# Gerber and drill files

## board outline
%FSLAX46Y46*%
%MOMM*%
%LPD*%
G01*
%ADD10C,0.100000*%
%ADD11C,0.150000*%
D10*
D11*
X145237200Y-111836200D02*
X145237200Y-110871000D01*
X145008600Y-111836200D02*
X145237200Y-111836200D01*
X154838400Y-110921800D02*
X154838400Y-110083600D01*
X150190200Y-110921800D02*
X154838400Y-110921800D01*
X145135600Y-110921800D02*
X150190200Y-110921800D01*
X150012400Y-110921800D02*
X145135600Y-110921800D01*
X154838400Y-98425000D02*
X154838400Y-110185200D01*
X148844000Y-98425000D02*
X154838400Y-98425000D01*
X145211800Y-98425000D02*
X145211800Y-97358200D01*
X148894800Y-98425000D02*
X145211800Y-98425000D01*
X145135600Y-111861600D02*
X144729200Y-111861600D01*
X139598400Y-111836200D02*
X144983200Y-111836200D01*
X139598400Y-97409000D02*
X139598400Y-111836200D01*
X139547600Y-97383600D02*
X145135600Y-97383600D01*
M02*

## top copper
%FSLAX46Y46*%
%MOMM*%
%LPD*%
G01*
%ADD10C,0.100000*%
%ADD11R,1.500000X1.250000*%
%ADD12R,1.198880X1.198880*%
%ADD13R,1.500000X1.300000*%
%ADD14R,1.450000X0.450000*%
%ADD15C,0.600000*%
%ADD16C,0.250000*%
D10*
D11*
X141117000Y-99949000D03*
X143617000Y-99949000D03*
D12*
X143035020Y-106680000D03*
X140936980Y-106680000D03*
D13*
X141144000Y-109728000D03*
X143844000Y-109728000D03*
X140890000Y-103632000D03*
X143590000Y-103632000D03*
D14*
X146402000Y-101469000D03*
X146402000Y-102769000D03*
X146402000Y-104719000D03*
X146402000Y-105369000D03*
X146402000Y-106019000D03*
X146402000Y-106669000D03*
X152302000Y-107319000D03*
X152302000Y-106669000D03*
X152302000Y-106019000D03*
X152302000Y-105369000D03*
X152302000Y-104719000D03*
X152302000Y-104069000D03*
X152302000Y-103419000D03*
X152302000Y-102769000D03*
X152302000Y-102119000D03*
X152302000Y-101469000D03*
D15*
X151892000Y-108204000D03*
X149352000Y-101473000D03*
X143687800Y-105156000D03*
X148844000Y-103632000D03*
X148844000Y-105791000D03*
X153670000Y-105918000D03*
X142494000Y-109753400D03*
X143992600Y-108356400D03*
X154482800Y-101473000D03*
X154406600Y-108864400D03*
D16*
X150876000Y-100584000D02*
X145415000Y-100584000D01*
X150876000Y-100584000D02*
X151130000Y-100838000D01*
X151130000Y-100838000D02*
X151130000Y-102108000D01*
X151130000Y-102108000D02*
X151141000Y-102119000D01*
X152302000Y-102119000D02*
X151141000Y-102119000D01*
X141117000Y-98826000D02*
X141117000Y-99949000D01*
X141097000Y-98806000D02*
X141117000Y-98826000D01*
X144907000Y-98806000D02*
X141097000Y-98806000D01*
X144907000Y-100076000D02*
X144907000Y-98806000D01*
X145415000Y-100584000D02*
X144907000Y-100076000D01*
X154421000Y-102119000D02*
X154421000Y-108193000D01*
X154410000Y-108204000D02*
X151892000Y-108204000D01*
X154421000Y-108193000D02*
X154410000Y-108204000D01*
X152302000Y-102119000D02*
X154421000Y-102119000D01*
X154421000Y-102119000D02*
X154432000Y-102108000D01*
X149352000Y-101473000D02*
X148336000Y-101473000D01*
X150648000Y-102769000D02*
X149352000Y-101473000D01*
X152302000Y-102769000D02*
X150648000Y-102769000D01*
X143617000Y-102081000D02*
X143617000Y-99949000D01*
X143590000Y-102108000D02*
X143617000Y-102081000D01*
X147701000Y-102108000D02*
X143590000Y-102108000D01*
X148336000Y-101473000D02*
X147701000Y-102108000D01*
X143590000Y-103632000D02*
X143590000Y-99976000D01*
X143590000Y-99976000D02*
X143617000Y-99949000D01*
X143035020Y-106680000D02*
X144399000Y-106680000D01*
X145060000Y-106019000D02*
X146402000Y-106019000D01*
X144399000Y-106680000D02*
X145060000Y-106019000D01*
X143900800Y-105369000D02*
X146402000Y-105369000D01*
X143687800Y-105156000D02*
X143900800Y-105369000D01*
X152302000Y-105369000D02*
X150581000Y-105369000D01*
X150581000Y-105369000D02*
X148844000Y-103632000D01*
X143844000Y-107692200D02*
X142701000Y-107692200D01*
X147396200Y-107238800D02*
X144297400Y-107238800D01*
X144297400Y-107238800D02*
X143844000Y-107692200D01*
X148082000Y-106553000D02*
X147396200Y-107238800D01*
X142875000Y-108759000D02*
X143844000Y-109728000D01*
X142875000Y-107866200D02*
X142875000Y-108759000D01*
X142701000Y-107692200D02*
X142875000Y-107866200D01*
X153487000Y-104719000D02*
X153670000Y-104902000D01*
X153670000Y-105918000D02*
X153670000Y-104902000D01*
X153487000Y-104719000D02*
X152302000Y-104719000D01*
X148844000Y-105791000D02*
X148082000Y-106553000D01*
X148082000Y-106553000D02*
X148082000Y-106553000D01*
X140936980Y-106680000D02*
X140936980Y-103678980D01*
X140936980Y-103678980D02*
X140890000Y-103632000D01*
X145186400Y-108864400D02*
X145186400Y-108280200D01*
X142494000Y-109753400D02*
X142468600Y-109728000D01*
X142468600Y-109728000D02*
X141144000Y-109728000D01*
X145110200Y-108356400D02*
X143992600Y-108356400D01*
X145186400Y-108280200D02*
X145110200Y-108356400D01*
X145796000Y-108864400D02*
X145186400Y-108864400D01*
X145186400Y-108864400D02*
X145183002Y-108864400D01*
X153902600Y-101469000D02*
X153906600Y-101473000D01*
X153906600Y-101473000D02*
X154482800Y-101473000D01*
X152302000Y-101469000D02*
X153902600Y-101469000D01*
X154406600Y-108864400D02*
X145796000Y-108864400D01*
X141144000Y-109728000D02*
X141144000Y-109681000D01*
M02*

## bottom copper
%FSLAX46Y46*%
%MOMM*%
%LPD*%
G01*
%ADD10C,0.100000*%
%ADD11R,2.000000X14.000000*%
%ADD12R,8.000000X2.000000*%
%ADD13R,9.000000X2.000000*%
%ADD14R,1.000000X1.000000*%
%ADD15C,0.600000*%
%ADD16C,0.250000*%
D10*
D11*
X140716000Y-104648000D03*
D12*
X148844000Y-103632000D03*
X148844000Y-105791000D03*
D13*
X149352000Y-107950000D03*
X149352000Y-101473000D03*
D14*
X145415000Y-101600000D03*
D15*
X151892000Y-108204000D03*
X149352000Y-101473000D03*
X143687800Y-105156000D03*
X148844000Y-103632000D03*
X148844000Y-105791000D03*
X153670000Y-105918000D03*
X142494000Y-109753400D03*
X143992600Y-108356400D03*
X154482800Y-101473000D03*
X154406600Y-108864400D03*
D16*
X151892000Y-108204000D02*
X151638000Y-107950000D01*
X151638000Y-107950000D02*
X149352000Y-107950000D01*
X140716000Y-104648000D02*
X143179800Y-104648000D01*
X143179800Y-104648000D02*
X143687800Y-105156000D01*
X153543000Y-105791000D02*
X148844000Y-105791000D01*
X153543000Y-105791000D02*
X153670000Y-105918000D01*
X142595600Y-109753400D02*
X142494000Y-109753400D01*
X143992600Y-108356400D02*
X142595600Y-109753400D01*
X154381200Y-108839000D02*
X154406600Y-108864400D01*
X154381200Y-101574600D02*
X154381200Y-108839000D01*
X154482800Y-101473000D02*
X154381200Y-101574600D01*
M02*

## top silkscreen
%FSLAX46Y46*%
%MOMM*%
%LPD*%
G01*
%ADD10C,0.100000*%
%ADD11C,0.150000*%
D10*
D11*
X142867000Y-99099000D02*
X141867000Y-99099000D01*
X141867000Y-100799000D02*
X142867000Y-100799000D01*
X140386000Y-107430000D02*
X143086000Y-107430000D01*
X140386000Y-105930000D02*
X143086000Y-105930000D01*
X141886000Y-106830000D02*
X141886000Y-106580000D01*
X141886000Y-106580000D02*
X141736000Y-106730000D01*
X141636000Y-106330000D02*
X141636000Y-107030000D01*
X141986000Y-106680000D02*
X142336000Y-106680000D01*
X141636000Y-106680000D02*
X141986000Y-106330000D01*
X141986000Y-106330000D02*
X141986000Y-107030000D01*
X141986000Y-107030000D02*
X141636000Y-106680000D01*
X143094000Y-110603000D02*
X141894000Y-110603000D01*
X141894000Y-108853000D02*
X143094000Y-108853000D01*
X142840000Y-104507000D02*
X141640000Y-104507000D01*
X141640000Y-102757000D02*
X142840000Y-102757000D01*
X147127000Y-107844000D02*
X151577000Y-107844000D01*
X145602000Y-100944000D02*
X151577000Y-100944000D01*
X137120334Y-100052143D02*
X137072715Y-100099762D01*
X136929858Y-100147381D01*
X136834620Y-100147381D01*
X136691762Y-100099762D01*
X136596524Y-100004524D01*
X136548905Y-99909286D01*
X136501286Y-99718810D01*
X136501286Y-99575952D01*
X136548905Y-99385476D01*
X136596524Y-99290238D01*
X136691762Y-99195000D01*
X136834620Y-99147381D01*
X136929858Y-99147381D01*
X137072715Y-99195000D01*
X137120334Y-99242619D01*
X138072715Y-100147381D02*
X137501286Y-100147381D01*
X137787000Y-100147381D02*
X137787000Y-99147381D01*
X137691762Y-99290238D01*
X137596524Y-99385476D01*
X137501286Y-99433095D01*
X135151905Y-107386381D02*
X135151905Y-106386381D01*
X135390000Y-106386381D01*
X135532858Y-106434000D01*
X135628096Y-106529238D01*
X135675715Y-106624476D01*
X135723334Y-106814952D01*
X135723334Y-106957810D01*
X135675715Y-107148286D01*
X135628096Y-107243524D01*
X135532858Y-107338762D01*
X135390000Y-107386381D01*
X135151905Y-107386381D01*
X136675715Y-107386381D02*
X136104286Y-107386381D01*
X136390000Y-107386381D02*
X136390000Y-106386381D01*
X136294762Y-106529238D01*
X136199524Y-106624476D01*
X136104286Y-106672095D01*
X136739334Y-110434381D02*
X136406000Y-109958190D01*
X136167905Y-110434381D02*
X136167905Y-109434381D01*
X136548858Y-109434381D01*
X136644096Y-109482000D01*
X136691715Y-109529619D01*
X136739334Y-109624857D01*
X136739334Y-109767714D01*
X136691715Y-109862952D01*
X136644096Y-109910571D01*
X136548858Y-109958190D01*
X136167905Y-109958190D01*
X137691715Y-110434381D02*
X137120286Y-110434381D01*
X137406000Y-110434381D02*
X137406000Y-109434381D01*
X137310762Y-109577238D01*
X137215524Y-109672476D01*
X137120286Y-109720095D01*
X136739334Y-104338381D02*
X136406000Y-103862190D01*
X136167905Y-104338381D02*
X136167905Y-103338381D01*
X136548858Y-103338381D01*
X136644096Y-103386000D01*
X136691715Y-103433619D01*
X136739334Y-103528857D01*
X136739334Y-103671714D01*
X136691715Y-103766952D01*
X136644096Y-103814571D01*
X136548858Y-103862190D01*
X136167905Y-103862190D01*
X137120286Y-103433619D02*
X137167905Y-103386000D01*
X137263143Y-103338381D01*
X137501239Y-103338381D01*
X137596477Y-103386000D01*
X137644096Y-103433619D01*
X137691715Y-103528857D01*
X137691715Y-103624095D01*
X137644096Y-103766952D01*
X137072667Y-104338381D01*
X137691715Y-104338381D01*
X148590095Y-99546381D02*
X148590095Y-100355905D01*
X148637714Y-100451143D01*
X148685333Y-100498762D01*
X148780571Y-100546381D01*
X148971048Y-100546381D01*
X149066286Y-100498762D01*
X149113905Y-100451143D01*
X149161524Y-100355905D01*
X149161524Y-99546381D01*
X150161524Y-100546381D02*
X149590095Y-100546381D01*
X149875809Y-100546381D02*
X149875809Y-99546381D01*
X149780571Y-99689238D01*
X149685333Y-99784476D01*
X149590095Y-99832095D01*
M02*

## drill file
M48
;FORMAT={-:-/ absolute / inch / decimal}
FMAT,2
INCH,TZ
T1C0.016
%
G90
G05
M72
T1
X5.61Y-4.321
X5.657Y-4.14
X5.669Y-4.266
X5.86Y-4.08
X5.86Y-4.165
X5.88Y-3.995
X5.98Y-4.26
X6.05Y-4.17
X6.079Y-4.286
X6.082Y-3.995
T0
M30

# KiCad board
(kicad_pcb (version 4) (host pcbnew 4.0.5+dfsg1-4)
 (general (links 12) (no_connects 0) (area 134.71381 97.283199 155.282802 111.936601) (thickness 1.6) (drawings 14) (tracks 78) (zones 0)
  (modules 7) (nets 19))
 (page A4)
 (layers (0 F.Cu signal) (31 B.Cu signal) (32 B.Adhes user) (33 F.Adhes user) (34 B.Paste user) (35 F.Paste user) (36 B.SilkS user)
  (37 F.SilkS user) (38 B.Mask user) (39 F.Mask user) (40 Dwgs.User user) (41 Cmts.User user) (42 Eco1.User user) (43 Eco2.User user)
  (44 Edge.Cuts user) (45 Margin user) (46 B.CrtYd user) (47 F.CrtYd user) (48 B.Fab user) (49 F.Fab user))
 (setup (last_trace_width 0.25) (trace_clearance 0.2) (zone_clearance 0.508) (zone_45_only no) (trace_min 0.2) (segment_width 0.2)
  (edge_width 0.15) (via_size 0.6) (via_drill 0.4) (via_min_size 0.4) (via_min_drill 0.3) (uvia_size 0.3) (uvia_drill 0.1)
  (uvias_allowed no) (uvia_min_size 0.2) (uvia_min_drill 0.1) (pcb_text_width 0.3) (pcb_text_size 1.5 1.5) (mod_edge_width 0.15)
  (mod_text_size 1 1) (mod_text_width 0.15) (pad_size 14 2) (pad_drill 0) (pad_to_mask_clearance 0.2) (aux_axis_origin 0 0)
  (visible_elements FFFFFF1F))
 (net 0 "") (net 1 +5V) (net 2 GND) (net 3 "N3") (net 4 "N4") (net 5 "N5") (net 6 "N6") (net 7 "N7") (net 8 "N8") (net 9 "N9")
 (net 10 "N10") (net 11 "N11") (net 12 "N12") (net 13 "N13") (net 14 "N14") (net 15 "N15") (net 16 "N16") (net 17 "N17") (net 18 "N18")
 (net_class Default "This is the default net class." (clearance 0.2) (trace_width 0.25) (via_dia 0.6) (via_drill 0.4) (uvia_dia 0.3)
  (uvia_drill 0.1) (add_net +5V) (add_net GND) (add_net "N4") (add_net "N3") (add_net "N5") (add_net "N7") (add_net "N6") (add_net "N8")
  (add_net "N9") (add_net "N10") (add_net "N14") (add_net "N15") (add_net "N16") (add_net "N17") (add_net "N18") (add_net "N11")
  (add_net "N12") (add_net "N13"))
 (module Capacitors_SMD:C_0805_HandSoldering (layer F.Cu) (at 142.367 99.949)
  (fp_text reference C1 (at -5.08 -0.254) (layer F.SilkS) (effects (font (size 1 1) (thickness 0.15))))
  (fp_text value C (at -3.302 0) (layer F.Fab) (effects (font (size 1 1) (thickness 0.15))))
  (fp_line (start 0.5 -0.85) (end -0.5 -0.85) (layer F.SilkS) (width 0.15))
  (fp_line (start -0.5 0.85) (end 0.5 0.85) (layer F.SilkS) (width 0.15))
  (pad 1 smd rect (at -1.25 0) (size 1.5 1.25) (layers F.Cu F.Paste F.Mask) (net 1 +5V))
  (pad 2 smd rect (at 1.25 0) (size 1.5 1.25) (layers F.Cu F.Paste F.Mask) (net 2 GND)))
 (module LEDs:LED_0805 (layer F.Cu) (at 141.986 106.68)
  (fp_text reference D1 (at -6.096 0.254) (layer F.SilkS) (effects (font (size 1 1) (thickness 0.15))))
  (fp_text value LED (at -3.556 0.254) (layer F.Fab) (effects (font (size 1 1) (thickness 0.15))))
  (fp_line (start -1.6 0.75) (end 1.1 0.75) (layer F.SilkS) (width 0.15))
  (fp_line (start -1.6 -0.75) (end 1.1 -0.75) (layer F.SilkS) (width 0.15))
  (fp_line (start -0.1 0.15) (end -0.1 -0.1) (layer F.SilkS) (width 0.15))
  (fp_line (start -0.1 -0.1) (end -0.25 0.05) (layer F.SilkS) (width 0.15))
  (fp_line (start -0.35 -0.35) (end -0.35 0.35) (layer F.SilkS) (width 0.15))
  (fp_line (start 0 0) (end 0.35 0) (layer F.SilkS) (width 0.15))
  (fp_line (start -0.35 0) (end 0 -0.35) (layer F.SilkS) (width 0.15))
  (fp_line (start 0 -0.35) (end 0 0.35) (layer F.SilkS) (width 0.15))
  (fp_line (start 0 0.35) (end -0.35 0) (layer F.SilkS) (width 0.15))
  (pad 2 smd rect (at 1.04902 0 180) (size 1.19888 1.19888) (layers F.Cu F.Paste F.Mask) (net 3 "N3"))
  (pad 1 smd rect (at -1.04902 0 180) (size 1.19888 1.19888) (layers F.Cu F.Paste F.Mask) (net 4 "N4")))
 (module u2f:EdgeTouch (layer B.Cu) (at 140.716 104.648 270)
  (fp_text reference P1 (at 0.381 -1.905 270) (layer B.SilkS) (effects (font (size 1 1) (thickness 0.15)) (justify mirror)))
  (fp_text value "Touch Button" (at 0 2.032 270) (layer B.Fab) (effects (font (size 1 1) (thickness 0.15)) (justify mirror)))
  (pad 1 connect rect (at 0 0 270) (size 14 2) (layers B.Cu B.Mask) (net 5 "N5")))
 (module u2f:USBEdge (layer B.Cu) (at 148.844 104.648)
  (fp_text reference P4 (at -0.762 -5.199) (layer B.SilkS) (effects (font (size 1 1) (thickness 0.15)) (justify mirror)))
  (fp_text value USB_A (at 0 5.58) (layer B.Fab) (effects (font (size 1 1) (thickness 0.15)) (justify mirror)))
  (pad 3 connect rect (at 0 -1.016) (size 8 2) (layers B.Cu B.Mask) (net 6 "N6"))
  (pad 2 connect rect (at 0 1.143) (size 8 2) (layers B.Cu B.Mask) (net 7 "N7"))
  (pad 1 connect rect (at 0.508 3.302) (size 9 2) (layers B.Cu B.Mask) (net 1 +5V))
  (pad 4 connect rect (at 0.508 -3.175) (size 9 2) (layers B.Cu B.Mask) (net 2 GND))
  (pad 5 connect rect (at -3.429 -3.048) (size 1 1) (layers B.Cu B.Mask) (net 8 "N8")))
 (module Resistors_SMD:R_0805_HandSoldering (layer F.Cu) (at 142.494 109.728)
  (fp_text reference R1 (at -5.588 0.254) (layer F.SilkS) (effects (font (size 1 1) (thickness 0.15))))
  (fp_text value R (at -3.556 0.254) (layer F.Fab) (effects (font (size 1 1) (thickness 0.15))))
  (fp_line (start 0.6 0.875) (end -0.6 0.875) (layer F.SilkS) (width 0.15))
  (fp_line (start -0.6 -0.875) (end 0.6 -0.875) (layer F.SilkS) (width 0.15))
  (pad 1 smd rect (at -1.35 0) (size 1.5 1.3) (layers F.Cu F.Paste F.Mask) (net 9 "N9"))
  (pad 2 smd rect (at 1.35 0) (size 1.5 1.3) (layers F.Cu F.Paste F.Mask) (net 7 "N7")))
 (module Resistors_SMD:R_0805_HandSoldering (layer F.Cu) (at 142.24 103.632)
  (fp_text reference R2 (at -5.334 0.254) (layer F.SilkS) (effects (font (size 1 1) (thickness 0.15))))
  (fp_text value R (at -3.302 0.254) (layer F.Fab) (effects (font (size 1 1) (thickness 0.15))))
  (fp_line (start 0.6 0.875) (end -0.6 0.875) (layer F.SilkS) (width 0.15))
  (fp_line (start -0.6 -0.875) (end 0.6 -0.875) (layer F.SilkS) (width 0.15))
  (pad 1 smd rect (at -1.35 0) (size 1.5 1.3) (layers F.Cu F.Paste F.Mask) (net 4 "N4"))
  (pad 2 smd rect (at 1.35 0) (size 1.5 1.3) (layers F.Cu F.Paste F.Mask) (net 2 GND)))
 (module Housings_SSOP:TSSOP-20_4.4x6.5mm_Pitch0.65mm (layer F.Cu) (at 149.352 104.394)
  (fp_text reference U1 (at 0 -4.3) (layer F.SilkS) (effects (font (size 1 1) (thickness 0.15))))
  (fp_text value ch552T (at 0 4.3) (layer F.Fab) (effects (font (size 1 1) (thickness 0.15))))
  (fp_line (start -2.225 3.45) (end 2.225 3.45) (layer F.SilkS) (width 0.15))
  (fp_line (start -3.75 -3.45) (end 2.225 -3.45) (layer F.SilkS) (width 0.15))
  (pad 1 smd rect (at -2.95 -2.925) (size 1.45 0.45) (layers F.Cu F.Paste F.Mask) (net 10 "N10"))
  (pad 3 smd rect (at -2.95 -1.625) (size 1.45 0.45) (layers F.Cu F.Paste F.Mask) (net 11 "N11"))
  (pad 6 smd rect (at -2.95 0.325) (size 1.45 0.45) (layers F.Cu F.Paste F.Mask) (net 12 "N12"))
  (pad 7 smd rect (at -2.95 0.975) (size 1.45 0.45) (layers F.Cu F.Paste F.Mask) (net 5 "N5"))
  (pad 8 smd rect (at -2.95 1.625) (size 1.45 0.45) (layers F.Cu F.Paste F.Mask) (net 3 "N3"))
  (pad 9 smd rect (at -2.95 2.275) (size 1.45 0.45) (layers F.Cu F.Paste F.Mask) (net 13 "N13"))
  (pad 11 smd rect (at 2.95 2.925) (size 1.45 0.45) (layers F.Cu F.Paste F.Mask) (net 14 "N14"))
  (pad 12 smd rect (at 2.95 2.275) (size 1.45 0.45) (layers F.Cu F.Paste F.Mask) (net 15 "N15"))
  (pad 13 smd rect (at 2.95 1.625) (size 1.45 0.45) (layers F.Cu F.Paste F.Mask) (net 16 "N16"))
  (pad 14 smd rect (at 2.95 0.975) (size 1.45 0.45) (layers F.Cu F.Paste F.Mask) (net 6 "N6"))
  (pad 15 smd rect (at 2.95 0.325) (size 1.45 0.45) (layers F.Cu F.Paste F.Mask) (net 7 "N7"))
  (pad 16 smd rect (at 2.95 -0.325) (size 1.45 0.45) (layers F.Cu F.Paste F.Mask) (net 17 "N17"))
  (pad 17 smd rect (at 2.95 -0.975) (size 1.45 0.45) (layers F.Cu F.Paste F.Mask) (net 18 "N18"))
  (pad 18 smd rect (at 2.95 -1.625) (size 1.45 0.45) (layers F.Cu F.Paste F.Mask) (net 2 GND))
  (pad 19 smd rect (at 2.95 -2.275) (size 1.45 0.45) (layers F.Cu F.Paste F.Mask) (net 1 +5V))
  (pad 20 smd rect (at 2.95 -2.925) (size 1.45 0.45) (layers F.Cu F.Paste F.Mask) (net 9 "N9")))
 (gr_line (start 145.2372 111.8362) (end 145.2372 110.871) (angle 90) (layer Edge.Cuts) (width 0.15))
 (gr_line (start 145.0086 111.8362) (end 145.2372 111.8362) (angle 90) (layer Edge.Cuts) (width 0.15))
 (gr_line (start 154.8384 110.9218) (end 154.8384 110.0836) (angle 90) (layer Edge.Cuts) (width 0.15))
 (gr_line (start 150.1902 110.9218) (end 154.8384 110.9218) (angle 90) (layer Edge.Cuts) (width 0.15))
 (gr_line (start 145.1356 110.9218) (end 150.1902 110.9218) (angle 90) (layer Edge.Cuts) (width 0.15))
 (gr_line (start 150.0124 110.9218) (end 145.1356 110.9218) (angle 90) (layer Edge.Cuts) (width 0.15))
 (gr_line (start 154.8384 98.425) (end 154.8384 110.1852) (angle 90) (layer Edge.Cuts) (width 0.15))
 (gr_line (start 148.844 98.425) (end 154.8384 98.425) (angle 90) (layer Edge.Cuts) (width 0.15))
 (gr_line (start 145.2118 98.425) (end 145.2118 97.3582) (angle 90) (layer Edge.Cuts) (width 0.15))
 (gr_line (start 148.8948 98.425) (end 145.2118 98.425) (angle 90) (layer Edge.Cuts) (width 0.15))
 (gr_line (start 145.1356 111.8616) (end 144.7292 111.8616) (angle 90) (layer Edge.Cuts) (width 0.15))
 (gr_line (start 139.5984 111.8362) (end 144.9832 111.8362) (angle 90) (layer Edge.Cuts) (width 0.15))
 (gr_line (start 139.5984 97.409) (end 139.5984 111.8362) (angle 90) (layer Edge.Cuts) (width 0.15))
 (gr_line (start 139.5476 97.3836) (end 145.1356 97.3836) (angle 90) (layer Edge.Cuts) (width 0.15))
 (segment (start 150.876 100.584) (end 145.415 100.584) (width 0.25) (layer F.Cu) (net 1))
 (segment (start 150.876 100.584) (end 151.13 100.838) (width 0.25) (layer F.Cu) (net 1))
 (segment (start 151.13 100.838) (end 151.13 102.108) (width 0.25) (layer F.Cu) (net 1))
 (segment (start 151.13 102.108) (end 151.141 102.119) (width 0.25) (layer F.Cu) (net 1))
 (segment (start 152.302 102.119) (end 151.141 102.119) (width 0.25) (layer F.Cu) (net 1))
 (segment (start 141.117 98.826) (end 141.117 99.949) (width 0.25) (layer F.Cu) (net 1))
 (segment (start 141.097 98.806) (end 141.117 98.826) (width 0.25) (layer F.Cu) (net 1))
 (segment (start 144.907 98.806) (end 141.097 98.806) (width 0.25) (layer F.Cu) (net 1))
 (segment (start 144.907 100.076) (end 144.907 98.806) (width 0.25) (layer F.Cu) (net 1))
 (segment (start 145.415 100.584) (end 144.907 100.076) (width 0.25) (layer F.Cu) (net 1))
 (segment (start 154.421 102.119) (end 154.421 108.193) (width 0.25) (layer F.Cu) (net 1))
 (segment (start 151.892 108.204) (end 151.638 107.95) (width 0.25) (layer B.Cu) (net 1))
 (via (at 151.892 108.204) (size 0.6) (drill 0.4) (layers F.Cu B.Cu) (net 1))
 (segment (start 154.41 108.204) (end 151.892 108.204) (width 0.25) (layer F.Cu) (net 1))
 (segment (start 154.421 108.193) (end 154.41 108.204) (width 0.25) (layer F.Cu) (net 1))
 (segment (start 151.638 107.95) (end 149.352 107.95) (width 0.25) (layer B.Cu) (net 1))
 (segment (start 152.302 102.119) (end 154.421 102.119) (width 0.25) (layer F.Cu) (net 1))
 (segment (start 154.421 102.119) (end 154.432 102.108) (width 0.25) (layer F.Cu) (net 1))
 (segment (start 149.352 101.473) (end 148.336 101.473) (width 0.25) (layer F.Cu) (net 2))
 (segment (start 150.648 102.769) (end 149.352 101.473) (width 0.25) (layer F.Cu) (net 2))
 (segment (start 152.302 102.769) (end 150.648 102.769) (width 0.25) (layer F.Cu) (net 2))
 (via (at 149.352 101.473) (size 0.6) (drill 0.4) (layers F.Cu B.Cu) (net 2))
 (segment (start 143.617 102.081) (end 143.617 99.949) (width 0.25) (layer F.Cu) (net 2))
 (segment (start 143.59 102.108) (end 143.617 102.081) (width 0.25) (layer F.Cu) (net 2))
 (segment (start 147.701 102.108) (end 143.59 102.108) (width 0.25) (layer F.Cu) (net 2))
 (segment (start 148.336 101.473) (end 147.701 102.108) (width 0.25) (layer F.Cu) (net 2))
 (segment (start 143.59 103.632) (end 143.59 99.976) (width 0.25) (layer F.Cu) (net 2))
 (segment (start 143.59 99.976) (end 143.617 99.949) (width 0.25) (layer F.Cu) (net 2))
 (segment (start 143.03502 106.68) (end 144.399 106.68) (width 0.25) (layer F.Cu) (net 3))
 (segment (start 145.06 106.019) (end 146.402 106.019) (width 0.25) (layer F.Cu) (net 3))
 (segment (start 144.399 106.68) (end 145.06 106.019) (width 0.25) (layer F.Cu) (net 3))
 (segment (start 140.716 104.648) (end 143.1798 104.648) (width 0.25) (layer B.Cu) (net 5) (status 400000))
 (segment (start 143.9008 105.369) (end 146.402 105.369) (width 0.25) (layer F.Cu) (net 5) (status 800000))
 (segment (start 143.6878 105.156) (end 143.9008 105.369) (width 0.25) (layer F.Cu) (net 5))
 (via (at 143.6878 105.156) (size 0.6) (drill 0.4) (layers F.Cu B.Cu) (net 5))
 (segment (start 143.1798 104.648) (end 143.6878 105.156) (width 0.25) (layer B.Cu) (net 5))
 (via (at 148.844 103.632) (size 0.6) (drill 0.4) (layers F.Cu B.Cu) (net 6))
 (segment (start 152.302 105.369) (end 150.581 105.369) (width 0.25) (layer F.Cu) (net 6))
 (segment (start 150.581 105.369) (end 148.844 103.632) (width 0.25) (layer F.Cu) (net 6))
 (segment (start 143.844 107.6922) (end 142.701 107.6922) (width 0.25) (layer F.Cu) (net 7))
 (segment (start 147.3962 107.2388) (end 144.2974 107.2388) (width 0.25) (layer F.Cu) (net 7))
 (segment (start 144.2974 107.2388) (end 143.844 107.6922) (width 0.25) (layer F.Cu) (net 7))
 (segment (start 148.082 106.553) (end 147.3962 107.2388) (width 0.25) (layer F.Cu) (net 7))
 (segment (start 142.875 108.759) (end 143.844 109.728) (width 0.25) (layer F.Cu) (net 7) (status 800000))
 (segment (start 142.875 107.8662) (end 142.875 108.759) (width 0.25) (layer F.Cu) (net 7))
 (segment (start 142.701 107.6922) (end 142.875 107.8662) (width 0.25) (layer F.Cu) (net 7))
 (via (at 148.844 105.791) (size 0.6) (drill 0.4) (layers F.Cu B.Cu) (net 7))
 (segment (start 153.487 104.719) (end 153.67 104.902) (width 0.25) (layer F.Cu) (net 7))
 (segment (start 153.543 105.791) (end 148.844 105.791) (width 0.25) (layer B.Cu) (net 7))
 (segment (start 153.67 105.918) (end 153.67 104.902) (width 0.25) (layer F.Cu) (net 7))
 (via (at 153.67 105.918) (size 0.6) (drill 0.4) (layers F.Cu B.Cu) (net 7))
 (segment (start 153.543 105.791) (end 153.67 105.918) (width 0.25) (layer B.Cu) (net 7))
 (segment (start 153.487 104.719) (end 152.302 104.719) (width 0.25) (layer F.Cu) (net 7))
 (segment (start 148.844 105.791) (end 148.082 106.553) (width 0.25) (layer F.Cu) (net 7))
 (segment (start 148.082 106.553) (end 148.082 106.553) (width 0.25) (layer F.Cu) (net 7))
 (segment (start 140.93698 106.68) (end 140.93698 103.67898) (width 0.25) (layer F.Cu) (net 4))
 (segment (start 140.93698 103.67898) (end 140.89 103.632) (width 0.25) (layer F.Cu) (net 4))
 (segment (start 145.1864 108.8644) (end 145.1864 108.2802) (width 0.25) (layer F.Cu) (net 9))
 (via (at 142.494 109.7534) (size 0.6) (drill 0.4) (layers F.Cu B.Cu) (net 9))
 (segment (start 142.494 109.7534) (end 142.4686 109.728) (width 0.25) (layer F.Cu) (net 9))
 (segment (start 142.4686 109.728) (end 141.144 109.728) (width 0.25) (layer F.Cu) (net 9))
 (segment (start 142.5956 109.7534) (end 142.494 109.7534) (width 0.25) (layer B.Cu) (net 9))
 (segment (start 143.9926 108.3564) (end 142.5956 109.7534) (width 0.25) (layer B.Cu) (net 9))
 (via (at 143.9926 108.3564) (size 0.6) (drill 0.4) (layers F.Cu B.Cu) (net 9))
 (segment (start 145.1102 108.3564) (end 143.9926 108.3564) (width 0.25) (layer F.Cu) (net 9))
 (segment (start 145.1864 108.2802) (end 145.1102 108.3564) (width 0.25) (layer F.Cu) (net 9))
 (segment (start 145.796 108.8644) (end 145.1864 108.8644) (width 0.25) (layer F.Cu) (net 9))
 (segment (start 145.1864 108.8644) (end 145.183002 108.8644) (width 0.25) (layer F.Cu) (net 9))
 (via (at 154.4828 101.473) (size 0.6) (drill 0.4) (layers F.Cu B.Cu) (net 9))
 (segment (start 153.9026 101.469) (end 153.9066 101.473) (width 0.25) (layer F.Cu) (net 9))
 (segment (start 153.9066 101.473) (end 154.4828 101.473) (width 0.25) (layer F.Cu) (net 9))
 (segment (start 152.302 101.469) (end 153.9026 101.469) (width 0.25) (layer F.Cu) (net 9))
 (segment (start 154.4066 108.8644) (end 145.796 108.8644) (width 0.25) (layer F.Cu) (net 9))
 (via (at 154.4066 108.8644) (size 0.6) (drill 0.4) (layers F.Cu B.Cu) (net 9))
 (segment (start 154.3812 108.839) (end 154.4066 108.8644) (width 0.25) (layer B.Cu) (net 9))
 (segment (start 154.3812 101.5746) (end 154.3812 108.839) (width 0.25) (layer B.Cu) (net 9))
 (segment (start 154.4828 101.473) (end 154.3812 101.5746) (width 0.25) (layer B.Cu) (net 9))
 (segment (start 141.144 109.728) (end 141.144 109.681) (width 0.25) (layer F.Cu) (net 9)))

